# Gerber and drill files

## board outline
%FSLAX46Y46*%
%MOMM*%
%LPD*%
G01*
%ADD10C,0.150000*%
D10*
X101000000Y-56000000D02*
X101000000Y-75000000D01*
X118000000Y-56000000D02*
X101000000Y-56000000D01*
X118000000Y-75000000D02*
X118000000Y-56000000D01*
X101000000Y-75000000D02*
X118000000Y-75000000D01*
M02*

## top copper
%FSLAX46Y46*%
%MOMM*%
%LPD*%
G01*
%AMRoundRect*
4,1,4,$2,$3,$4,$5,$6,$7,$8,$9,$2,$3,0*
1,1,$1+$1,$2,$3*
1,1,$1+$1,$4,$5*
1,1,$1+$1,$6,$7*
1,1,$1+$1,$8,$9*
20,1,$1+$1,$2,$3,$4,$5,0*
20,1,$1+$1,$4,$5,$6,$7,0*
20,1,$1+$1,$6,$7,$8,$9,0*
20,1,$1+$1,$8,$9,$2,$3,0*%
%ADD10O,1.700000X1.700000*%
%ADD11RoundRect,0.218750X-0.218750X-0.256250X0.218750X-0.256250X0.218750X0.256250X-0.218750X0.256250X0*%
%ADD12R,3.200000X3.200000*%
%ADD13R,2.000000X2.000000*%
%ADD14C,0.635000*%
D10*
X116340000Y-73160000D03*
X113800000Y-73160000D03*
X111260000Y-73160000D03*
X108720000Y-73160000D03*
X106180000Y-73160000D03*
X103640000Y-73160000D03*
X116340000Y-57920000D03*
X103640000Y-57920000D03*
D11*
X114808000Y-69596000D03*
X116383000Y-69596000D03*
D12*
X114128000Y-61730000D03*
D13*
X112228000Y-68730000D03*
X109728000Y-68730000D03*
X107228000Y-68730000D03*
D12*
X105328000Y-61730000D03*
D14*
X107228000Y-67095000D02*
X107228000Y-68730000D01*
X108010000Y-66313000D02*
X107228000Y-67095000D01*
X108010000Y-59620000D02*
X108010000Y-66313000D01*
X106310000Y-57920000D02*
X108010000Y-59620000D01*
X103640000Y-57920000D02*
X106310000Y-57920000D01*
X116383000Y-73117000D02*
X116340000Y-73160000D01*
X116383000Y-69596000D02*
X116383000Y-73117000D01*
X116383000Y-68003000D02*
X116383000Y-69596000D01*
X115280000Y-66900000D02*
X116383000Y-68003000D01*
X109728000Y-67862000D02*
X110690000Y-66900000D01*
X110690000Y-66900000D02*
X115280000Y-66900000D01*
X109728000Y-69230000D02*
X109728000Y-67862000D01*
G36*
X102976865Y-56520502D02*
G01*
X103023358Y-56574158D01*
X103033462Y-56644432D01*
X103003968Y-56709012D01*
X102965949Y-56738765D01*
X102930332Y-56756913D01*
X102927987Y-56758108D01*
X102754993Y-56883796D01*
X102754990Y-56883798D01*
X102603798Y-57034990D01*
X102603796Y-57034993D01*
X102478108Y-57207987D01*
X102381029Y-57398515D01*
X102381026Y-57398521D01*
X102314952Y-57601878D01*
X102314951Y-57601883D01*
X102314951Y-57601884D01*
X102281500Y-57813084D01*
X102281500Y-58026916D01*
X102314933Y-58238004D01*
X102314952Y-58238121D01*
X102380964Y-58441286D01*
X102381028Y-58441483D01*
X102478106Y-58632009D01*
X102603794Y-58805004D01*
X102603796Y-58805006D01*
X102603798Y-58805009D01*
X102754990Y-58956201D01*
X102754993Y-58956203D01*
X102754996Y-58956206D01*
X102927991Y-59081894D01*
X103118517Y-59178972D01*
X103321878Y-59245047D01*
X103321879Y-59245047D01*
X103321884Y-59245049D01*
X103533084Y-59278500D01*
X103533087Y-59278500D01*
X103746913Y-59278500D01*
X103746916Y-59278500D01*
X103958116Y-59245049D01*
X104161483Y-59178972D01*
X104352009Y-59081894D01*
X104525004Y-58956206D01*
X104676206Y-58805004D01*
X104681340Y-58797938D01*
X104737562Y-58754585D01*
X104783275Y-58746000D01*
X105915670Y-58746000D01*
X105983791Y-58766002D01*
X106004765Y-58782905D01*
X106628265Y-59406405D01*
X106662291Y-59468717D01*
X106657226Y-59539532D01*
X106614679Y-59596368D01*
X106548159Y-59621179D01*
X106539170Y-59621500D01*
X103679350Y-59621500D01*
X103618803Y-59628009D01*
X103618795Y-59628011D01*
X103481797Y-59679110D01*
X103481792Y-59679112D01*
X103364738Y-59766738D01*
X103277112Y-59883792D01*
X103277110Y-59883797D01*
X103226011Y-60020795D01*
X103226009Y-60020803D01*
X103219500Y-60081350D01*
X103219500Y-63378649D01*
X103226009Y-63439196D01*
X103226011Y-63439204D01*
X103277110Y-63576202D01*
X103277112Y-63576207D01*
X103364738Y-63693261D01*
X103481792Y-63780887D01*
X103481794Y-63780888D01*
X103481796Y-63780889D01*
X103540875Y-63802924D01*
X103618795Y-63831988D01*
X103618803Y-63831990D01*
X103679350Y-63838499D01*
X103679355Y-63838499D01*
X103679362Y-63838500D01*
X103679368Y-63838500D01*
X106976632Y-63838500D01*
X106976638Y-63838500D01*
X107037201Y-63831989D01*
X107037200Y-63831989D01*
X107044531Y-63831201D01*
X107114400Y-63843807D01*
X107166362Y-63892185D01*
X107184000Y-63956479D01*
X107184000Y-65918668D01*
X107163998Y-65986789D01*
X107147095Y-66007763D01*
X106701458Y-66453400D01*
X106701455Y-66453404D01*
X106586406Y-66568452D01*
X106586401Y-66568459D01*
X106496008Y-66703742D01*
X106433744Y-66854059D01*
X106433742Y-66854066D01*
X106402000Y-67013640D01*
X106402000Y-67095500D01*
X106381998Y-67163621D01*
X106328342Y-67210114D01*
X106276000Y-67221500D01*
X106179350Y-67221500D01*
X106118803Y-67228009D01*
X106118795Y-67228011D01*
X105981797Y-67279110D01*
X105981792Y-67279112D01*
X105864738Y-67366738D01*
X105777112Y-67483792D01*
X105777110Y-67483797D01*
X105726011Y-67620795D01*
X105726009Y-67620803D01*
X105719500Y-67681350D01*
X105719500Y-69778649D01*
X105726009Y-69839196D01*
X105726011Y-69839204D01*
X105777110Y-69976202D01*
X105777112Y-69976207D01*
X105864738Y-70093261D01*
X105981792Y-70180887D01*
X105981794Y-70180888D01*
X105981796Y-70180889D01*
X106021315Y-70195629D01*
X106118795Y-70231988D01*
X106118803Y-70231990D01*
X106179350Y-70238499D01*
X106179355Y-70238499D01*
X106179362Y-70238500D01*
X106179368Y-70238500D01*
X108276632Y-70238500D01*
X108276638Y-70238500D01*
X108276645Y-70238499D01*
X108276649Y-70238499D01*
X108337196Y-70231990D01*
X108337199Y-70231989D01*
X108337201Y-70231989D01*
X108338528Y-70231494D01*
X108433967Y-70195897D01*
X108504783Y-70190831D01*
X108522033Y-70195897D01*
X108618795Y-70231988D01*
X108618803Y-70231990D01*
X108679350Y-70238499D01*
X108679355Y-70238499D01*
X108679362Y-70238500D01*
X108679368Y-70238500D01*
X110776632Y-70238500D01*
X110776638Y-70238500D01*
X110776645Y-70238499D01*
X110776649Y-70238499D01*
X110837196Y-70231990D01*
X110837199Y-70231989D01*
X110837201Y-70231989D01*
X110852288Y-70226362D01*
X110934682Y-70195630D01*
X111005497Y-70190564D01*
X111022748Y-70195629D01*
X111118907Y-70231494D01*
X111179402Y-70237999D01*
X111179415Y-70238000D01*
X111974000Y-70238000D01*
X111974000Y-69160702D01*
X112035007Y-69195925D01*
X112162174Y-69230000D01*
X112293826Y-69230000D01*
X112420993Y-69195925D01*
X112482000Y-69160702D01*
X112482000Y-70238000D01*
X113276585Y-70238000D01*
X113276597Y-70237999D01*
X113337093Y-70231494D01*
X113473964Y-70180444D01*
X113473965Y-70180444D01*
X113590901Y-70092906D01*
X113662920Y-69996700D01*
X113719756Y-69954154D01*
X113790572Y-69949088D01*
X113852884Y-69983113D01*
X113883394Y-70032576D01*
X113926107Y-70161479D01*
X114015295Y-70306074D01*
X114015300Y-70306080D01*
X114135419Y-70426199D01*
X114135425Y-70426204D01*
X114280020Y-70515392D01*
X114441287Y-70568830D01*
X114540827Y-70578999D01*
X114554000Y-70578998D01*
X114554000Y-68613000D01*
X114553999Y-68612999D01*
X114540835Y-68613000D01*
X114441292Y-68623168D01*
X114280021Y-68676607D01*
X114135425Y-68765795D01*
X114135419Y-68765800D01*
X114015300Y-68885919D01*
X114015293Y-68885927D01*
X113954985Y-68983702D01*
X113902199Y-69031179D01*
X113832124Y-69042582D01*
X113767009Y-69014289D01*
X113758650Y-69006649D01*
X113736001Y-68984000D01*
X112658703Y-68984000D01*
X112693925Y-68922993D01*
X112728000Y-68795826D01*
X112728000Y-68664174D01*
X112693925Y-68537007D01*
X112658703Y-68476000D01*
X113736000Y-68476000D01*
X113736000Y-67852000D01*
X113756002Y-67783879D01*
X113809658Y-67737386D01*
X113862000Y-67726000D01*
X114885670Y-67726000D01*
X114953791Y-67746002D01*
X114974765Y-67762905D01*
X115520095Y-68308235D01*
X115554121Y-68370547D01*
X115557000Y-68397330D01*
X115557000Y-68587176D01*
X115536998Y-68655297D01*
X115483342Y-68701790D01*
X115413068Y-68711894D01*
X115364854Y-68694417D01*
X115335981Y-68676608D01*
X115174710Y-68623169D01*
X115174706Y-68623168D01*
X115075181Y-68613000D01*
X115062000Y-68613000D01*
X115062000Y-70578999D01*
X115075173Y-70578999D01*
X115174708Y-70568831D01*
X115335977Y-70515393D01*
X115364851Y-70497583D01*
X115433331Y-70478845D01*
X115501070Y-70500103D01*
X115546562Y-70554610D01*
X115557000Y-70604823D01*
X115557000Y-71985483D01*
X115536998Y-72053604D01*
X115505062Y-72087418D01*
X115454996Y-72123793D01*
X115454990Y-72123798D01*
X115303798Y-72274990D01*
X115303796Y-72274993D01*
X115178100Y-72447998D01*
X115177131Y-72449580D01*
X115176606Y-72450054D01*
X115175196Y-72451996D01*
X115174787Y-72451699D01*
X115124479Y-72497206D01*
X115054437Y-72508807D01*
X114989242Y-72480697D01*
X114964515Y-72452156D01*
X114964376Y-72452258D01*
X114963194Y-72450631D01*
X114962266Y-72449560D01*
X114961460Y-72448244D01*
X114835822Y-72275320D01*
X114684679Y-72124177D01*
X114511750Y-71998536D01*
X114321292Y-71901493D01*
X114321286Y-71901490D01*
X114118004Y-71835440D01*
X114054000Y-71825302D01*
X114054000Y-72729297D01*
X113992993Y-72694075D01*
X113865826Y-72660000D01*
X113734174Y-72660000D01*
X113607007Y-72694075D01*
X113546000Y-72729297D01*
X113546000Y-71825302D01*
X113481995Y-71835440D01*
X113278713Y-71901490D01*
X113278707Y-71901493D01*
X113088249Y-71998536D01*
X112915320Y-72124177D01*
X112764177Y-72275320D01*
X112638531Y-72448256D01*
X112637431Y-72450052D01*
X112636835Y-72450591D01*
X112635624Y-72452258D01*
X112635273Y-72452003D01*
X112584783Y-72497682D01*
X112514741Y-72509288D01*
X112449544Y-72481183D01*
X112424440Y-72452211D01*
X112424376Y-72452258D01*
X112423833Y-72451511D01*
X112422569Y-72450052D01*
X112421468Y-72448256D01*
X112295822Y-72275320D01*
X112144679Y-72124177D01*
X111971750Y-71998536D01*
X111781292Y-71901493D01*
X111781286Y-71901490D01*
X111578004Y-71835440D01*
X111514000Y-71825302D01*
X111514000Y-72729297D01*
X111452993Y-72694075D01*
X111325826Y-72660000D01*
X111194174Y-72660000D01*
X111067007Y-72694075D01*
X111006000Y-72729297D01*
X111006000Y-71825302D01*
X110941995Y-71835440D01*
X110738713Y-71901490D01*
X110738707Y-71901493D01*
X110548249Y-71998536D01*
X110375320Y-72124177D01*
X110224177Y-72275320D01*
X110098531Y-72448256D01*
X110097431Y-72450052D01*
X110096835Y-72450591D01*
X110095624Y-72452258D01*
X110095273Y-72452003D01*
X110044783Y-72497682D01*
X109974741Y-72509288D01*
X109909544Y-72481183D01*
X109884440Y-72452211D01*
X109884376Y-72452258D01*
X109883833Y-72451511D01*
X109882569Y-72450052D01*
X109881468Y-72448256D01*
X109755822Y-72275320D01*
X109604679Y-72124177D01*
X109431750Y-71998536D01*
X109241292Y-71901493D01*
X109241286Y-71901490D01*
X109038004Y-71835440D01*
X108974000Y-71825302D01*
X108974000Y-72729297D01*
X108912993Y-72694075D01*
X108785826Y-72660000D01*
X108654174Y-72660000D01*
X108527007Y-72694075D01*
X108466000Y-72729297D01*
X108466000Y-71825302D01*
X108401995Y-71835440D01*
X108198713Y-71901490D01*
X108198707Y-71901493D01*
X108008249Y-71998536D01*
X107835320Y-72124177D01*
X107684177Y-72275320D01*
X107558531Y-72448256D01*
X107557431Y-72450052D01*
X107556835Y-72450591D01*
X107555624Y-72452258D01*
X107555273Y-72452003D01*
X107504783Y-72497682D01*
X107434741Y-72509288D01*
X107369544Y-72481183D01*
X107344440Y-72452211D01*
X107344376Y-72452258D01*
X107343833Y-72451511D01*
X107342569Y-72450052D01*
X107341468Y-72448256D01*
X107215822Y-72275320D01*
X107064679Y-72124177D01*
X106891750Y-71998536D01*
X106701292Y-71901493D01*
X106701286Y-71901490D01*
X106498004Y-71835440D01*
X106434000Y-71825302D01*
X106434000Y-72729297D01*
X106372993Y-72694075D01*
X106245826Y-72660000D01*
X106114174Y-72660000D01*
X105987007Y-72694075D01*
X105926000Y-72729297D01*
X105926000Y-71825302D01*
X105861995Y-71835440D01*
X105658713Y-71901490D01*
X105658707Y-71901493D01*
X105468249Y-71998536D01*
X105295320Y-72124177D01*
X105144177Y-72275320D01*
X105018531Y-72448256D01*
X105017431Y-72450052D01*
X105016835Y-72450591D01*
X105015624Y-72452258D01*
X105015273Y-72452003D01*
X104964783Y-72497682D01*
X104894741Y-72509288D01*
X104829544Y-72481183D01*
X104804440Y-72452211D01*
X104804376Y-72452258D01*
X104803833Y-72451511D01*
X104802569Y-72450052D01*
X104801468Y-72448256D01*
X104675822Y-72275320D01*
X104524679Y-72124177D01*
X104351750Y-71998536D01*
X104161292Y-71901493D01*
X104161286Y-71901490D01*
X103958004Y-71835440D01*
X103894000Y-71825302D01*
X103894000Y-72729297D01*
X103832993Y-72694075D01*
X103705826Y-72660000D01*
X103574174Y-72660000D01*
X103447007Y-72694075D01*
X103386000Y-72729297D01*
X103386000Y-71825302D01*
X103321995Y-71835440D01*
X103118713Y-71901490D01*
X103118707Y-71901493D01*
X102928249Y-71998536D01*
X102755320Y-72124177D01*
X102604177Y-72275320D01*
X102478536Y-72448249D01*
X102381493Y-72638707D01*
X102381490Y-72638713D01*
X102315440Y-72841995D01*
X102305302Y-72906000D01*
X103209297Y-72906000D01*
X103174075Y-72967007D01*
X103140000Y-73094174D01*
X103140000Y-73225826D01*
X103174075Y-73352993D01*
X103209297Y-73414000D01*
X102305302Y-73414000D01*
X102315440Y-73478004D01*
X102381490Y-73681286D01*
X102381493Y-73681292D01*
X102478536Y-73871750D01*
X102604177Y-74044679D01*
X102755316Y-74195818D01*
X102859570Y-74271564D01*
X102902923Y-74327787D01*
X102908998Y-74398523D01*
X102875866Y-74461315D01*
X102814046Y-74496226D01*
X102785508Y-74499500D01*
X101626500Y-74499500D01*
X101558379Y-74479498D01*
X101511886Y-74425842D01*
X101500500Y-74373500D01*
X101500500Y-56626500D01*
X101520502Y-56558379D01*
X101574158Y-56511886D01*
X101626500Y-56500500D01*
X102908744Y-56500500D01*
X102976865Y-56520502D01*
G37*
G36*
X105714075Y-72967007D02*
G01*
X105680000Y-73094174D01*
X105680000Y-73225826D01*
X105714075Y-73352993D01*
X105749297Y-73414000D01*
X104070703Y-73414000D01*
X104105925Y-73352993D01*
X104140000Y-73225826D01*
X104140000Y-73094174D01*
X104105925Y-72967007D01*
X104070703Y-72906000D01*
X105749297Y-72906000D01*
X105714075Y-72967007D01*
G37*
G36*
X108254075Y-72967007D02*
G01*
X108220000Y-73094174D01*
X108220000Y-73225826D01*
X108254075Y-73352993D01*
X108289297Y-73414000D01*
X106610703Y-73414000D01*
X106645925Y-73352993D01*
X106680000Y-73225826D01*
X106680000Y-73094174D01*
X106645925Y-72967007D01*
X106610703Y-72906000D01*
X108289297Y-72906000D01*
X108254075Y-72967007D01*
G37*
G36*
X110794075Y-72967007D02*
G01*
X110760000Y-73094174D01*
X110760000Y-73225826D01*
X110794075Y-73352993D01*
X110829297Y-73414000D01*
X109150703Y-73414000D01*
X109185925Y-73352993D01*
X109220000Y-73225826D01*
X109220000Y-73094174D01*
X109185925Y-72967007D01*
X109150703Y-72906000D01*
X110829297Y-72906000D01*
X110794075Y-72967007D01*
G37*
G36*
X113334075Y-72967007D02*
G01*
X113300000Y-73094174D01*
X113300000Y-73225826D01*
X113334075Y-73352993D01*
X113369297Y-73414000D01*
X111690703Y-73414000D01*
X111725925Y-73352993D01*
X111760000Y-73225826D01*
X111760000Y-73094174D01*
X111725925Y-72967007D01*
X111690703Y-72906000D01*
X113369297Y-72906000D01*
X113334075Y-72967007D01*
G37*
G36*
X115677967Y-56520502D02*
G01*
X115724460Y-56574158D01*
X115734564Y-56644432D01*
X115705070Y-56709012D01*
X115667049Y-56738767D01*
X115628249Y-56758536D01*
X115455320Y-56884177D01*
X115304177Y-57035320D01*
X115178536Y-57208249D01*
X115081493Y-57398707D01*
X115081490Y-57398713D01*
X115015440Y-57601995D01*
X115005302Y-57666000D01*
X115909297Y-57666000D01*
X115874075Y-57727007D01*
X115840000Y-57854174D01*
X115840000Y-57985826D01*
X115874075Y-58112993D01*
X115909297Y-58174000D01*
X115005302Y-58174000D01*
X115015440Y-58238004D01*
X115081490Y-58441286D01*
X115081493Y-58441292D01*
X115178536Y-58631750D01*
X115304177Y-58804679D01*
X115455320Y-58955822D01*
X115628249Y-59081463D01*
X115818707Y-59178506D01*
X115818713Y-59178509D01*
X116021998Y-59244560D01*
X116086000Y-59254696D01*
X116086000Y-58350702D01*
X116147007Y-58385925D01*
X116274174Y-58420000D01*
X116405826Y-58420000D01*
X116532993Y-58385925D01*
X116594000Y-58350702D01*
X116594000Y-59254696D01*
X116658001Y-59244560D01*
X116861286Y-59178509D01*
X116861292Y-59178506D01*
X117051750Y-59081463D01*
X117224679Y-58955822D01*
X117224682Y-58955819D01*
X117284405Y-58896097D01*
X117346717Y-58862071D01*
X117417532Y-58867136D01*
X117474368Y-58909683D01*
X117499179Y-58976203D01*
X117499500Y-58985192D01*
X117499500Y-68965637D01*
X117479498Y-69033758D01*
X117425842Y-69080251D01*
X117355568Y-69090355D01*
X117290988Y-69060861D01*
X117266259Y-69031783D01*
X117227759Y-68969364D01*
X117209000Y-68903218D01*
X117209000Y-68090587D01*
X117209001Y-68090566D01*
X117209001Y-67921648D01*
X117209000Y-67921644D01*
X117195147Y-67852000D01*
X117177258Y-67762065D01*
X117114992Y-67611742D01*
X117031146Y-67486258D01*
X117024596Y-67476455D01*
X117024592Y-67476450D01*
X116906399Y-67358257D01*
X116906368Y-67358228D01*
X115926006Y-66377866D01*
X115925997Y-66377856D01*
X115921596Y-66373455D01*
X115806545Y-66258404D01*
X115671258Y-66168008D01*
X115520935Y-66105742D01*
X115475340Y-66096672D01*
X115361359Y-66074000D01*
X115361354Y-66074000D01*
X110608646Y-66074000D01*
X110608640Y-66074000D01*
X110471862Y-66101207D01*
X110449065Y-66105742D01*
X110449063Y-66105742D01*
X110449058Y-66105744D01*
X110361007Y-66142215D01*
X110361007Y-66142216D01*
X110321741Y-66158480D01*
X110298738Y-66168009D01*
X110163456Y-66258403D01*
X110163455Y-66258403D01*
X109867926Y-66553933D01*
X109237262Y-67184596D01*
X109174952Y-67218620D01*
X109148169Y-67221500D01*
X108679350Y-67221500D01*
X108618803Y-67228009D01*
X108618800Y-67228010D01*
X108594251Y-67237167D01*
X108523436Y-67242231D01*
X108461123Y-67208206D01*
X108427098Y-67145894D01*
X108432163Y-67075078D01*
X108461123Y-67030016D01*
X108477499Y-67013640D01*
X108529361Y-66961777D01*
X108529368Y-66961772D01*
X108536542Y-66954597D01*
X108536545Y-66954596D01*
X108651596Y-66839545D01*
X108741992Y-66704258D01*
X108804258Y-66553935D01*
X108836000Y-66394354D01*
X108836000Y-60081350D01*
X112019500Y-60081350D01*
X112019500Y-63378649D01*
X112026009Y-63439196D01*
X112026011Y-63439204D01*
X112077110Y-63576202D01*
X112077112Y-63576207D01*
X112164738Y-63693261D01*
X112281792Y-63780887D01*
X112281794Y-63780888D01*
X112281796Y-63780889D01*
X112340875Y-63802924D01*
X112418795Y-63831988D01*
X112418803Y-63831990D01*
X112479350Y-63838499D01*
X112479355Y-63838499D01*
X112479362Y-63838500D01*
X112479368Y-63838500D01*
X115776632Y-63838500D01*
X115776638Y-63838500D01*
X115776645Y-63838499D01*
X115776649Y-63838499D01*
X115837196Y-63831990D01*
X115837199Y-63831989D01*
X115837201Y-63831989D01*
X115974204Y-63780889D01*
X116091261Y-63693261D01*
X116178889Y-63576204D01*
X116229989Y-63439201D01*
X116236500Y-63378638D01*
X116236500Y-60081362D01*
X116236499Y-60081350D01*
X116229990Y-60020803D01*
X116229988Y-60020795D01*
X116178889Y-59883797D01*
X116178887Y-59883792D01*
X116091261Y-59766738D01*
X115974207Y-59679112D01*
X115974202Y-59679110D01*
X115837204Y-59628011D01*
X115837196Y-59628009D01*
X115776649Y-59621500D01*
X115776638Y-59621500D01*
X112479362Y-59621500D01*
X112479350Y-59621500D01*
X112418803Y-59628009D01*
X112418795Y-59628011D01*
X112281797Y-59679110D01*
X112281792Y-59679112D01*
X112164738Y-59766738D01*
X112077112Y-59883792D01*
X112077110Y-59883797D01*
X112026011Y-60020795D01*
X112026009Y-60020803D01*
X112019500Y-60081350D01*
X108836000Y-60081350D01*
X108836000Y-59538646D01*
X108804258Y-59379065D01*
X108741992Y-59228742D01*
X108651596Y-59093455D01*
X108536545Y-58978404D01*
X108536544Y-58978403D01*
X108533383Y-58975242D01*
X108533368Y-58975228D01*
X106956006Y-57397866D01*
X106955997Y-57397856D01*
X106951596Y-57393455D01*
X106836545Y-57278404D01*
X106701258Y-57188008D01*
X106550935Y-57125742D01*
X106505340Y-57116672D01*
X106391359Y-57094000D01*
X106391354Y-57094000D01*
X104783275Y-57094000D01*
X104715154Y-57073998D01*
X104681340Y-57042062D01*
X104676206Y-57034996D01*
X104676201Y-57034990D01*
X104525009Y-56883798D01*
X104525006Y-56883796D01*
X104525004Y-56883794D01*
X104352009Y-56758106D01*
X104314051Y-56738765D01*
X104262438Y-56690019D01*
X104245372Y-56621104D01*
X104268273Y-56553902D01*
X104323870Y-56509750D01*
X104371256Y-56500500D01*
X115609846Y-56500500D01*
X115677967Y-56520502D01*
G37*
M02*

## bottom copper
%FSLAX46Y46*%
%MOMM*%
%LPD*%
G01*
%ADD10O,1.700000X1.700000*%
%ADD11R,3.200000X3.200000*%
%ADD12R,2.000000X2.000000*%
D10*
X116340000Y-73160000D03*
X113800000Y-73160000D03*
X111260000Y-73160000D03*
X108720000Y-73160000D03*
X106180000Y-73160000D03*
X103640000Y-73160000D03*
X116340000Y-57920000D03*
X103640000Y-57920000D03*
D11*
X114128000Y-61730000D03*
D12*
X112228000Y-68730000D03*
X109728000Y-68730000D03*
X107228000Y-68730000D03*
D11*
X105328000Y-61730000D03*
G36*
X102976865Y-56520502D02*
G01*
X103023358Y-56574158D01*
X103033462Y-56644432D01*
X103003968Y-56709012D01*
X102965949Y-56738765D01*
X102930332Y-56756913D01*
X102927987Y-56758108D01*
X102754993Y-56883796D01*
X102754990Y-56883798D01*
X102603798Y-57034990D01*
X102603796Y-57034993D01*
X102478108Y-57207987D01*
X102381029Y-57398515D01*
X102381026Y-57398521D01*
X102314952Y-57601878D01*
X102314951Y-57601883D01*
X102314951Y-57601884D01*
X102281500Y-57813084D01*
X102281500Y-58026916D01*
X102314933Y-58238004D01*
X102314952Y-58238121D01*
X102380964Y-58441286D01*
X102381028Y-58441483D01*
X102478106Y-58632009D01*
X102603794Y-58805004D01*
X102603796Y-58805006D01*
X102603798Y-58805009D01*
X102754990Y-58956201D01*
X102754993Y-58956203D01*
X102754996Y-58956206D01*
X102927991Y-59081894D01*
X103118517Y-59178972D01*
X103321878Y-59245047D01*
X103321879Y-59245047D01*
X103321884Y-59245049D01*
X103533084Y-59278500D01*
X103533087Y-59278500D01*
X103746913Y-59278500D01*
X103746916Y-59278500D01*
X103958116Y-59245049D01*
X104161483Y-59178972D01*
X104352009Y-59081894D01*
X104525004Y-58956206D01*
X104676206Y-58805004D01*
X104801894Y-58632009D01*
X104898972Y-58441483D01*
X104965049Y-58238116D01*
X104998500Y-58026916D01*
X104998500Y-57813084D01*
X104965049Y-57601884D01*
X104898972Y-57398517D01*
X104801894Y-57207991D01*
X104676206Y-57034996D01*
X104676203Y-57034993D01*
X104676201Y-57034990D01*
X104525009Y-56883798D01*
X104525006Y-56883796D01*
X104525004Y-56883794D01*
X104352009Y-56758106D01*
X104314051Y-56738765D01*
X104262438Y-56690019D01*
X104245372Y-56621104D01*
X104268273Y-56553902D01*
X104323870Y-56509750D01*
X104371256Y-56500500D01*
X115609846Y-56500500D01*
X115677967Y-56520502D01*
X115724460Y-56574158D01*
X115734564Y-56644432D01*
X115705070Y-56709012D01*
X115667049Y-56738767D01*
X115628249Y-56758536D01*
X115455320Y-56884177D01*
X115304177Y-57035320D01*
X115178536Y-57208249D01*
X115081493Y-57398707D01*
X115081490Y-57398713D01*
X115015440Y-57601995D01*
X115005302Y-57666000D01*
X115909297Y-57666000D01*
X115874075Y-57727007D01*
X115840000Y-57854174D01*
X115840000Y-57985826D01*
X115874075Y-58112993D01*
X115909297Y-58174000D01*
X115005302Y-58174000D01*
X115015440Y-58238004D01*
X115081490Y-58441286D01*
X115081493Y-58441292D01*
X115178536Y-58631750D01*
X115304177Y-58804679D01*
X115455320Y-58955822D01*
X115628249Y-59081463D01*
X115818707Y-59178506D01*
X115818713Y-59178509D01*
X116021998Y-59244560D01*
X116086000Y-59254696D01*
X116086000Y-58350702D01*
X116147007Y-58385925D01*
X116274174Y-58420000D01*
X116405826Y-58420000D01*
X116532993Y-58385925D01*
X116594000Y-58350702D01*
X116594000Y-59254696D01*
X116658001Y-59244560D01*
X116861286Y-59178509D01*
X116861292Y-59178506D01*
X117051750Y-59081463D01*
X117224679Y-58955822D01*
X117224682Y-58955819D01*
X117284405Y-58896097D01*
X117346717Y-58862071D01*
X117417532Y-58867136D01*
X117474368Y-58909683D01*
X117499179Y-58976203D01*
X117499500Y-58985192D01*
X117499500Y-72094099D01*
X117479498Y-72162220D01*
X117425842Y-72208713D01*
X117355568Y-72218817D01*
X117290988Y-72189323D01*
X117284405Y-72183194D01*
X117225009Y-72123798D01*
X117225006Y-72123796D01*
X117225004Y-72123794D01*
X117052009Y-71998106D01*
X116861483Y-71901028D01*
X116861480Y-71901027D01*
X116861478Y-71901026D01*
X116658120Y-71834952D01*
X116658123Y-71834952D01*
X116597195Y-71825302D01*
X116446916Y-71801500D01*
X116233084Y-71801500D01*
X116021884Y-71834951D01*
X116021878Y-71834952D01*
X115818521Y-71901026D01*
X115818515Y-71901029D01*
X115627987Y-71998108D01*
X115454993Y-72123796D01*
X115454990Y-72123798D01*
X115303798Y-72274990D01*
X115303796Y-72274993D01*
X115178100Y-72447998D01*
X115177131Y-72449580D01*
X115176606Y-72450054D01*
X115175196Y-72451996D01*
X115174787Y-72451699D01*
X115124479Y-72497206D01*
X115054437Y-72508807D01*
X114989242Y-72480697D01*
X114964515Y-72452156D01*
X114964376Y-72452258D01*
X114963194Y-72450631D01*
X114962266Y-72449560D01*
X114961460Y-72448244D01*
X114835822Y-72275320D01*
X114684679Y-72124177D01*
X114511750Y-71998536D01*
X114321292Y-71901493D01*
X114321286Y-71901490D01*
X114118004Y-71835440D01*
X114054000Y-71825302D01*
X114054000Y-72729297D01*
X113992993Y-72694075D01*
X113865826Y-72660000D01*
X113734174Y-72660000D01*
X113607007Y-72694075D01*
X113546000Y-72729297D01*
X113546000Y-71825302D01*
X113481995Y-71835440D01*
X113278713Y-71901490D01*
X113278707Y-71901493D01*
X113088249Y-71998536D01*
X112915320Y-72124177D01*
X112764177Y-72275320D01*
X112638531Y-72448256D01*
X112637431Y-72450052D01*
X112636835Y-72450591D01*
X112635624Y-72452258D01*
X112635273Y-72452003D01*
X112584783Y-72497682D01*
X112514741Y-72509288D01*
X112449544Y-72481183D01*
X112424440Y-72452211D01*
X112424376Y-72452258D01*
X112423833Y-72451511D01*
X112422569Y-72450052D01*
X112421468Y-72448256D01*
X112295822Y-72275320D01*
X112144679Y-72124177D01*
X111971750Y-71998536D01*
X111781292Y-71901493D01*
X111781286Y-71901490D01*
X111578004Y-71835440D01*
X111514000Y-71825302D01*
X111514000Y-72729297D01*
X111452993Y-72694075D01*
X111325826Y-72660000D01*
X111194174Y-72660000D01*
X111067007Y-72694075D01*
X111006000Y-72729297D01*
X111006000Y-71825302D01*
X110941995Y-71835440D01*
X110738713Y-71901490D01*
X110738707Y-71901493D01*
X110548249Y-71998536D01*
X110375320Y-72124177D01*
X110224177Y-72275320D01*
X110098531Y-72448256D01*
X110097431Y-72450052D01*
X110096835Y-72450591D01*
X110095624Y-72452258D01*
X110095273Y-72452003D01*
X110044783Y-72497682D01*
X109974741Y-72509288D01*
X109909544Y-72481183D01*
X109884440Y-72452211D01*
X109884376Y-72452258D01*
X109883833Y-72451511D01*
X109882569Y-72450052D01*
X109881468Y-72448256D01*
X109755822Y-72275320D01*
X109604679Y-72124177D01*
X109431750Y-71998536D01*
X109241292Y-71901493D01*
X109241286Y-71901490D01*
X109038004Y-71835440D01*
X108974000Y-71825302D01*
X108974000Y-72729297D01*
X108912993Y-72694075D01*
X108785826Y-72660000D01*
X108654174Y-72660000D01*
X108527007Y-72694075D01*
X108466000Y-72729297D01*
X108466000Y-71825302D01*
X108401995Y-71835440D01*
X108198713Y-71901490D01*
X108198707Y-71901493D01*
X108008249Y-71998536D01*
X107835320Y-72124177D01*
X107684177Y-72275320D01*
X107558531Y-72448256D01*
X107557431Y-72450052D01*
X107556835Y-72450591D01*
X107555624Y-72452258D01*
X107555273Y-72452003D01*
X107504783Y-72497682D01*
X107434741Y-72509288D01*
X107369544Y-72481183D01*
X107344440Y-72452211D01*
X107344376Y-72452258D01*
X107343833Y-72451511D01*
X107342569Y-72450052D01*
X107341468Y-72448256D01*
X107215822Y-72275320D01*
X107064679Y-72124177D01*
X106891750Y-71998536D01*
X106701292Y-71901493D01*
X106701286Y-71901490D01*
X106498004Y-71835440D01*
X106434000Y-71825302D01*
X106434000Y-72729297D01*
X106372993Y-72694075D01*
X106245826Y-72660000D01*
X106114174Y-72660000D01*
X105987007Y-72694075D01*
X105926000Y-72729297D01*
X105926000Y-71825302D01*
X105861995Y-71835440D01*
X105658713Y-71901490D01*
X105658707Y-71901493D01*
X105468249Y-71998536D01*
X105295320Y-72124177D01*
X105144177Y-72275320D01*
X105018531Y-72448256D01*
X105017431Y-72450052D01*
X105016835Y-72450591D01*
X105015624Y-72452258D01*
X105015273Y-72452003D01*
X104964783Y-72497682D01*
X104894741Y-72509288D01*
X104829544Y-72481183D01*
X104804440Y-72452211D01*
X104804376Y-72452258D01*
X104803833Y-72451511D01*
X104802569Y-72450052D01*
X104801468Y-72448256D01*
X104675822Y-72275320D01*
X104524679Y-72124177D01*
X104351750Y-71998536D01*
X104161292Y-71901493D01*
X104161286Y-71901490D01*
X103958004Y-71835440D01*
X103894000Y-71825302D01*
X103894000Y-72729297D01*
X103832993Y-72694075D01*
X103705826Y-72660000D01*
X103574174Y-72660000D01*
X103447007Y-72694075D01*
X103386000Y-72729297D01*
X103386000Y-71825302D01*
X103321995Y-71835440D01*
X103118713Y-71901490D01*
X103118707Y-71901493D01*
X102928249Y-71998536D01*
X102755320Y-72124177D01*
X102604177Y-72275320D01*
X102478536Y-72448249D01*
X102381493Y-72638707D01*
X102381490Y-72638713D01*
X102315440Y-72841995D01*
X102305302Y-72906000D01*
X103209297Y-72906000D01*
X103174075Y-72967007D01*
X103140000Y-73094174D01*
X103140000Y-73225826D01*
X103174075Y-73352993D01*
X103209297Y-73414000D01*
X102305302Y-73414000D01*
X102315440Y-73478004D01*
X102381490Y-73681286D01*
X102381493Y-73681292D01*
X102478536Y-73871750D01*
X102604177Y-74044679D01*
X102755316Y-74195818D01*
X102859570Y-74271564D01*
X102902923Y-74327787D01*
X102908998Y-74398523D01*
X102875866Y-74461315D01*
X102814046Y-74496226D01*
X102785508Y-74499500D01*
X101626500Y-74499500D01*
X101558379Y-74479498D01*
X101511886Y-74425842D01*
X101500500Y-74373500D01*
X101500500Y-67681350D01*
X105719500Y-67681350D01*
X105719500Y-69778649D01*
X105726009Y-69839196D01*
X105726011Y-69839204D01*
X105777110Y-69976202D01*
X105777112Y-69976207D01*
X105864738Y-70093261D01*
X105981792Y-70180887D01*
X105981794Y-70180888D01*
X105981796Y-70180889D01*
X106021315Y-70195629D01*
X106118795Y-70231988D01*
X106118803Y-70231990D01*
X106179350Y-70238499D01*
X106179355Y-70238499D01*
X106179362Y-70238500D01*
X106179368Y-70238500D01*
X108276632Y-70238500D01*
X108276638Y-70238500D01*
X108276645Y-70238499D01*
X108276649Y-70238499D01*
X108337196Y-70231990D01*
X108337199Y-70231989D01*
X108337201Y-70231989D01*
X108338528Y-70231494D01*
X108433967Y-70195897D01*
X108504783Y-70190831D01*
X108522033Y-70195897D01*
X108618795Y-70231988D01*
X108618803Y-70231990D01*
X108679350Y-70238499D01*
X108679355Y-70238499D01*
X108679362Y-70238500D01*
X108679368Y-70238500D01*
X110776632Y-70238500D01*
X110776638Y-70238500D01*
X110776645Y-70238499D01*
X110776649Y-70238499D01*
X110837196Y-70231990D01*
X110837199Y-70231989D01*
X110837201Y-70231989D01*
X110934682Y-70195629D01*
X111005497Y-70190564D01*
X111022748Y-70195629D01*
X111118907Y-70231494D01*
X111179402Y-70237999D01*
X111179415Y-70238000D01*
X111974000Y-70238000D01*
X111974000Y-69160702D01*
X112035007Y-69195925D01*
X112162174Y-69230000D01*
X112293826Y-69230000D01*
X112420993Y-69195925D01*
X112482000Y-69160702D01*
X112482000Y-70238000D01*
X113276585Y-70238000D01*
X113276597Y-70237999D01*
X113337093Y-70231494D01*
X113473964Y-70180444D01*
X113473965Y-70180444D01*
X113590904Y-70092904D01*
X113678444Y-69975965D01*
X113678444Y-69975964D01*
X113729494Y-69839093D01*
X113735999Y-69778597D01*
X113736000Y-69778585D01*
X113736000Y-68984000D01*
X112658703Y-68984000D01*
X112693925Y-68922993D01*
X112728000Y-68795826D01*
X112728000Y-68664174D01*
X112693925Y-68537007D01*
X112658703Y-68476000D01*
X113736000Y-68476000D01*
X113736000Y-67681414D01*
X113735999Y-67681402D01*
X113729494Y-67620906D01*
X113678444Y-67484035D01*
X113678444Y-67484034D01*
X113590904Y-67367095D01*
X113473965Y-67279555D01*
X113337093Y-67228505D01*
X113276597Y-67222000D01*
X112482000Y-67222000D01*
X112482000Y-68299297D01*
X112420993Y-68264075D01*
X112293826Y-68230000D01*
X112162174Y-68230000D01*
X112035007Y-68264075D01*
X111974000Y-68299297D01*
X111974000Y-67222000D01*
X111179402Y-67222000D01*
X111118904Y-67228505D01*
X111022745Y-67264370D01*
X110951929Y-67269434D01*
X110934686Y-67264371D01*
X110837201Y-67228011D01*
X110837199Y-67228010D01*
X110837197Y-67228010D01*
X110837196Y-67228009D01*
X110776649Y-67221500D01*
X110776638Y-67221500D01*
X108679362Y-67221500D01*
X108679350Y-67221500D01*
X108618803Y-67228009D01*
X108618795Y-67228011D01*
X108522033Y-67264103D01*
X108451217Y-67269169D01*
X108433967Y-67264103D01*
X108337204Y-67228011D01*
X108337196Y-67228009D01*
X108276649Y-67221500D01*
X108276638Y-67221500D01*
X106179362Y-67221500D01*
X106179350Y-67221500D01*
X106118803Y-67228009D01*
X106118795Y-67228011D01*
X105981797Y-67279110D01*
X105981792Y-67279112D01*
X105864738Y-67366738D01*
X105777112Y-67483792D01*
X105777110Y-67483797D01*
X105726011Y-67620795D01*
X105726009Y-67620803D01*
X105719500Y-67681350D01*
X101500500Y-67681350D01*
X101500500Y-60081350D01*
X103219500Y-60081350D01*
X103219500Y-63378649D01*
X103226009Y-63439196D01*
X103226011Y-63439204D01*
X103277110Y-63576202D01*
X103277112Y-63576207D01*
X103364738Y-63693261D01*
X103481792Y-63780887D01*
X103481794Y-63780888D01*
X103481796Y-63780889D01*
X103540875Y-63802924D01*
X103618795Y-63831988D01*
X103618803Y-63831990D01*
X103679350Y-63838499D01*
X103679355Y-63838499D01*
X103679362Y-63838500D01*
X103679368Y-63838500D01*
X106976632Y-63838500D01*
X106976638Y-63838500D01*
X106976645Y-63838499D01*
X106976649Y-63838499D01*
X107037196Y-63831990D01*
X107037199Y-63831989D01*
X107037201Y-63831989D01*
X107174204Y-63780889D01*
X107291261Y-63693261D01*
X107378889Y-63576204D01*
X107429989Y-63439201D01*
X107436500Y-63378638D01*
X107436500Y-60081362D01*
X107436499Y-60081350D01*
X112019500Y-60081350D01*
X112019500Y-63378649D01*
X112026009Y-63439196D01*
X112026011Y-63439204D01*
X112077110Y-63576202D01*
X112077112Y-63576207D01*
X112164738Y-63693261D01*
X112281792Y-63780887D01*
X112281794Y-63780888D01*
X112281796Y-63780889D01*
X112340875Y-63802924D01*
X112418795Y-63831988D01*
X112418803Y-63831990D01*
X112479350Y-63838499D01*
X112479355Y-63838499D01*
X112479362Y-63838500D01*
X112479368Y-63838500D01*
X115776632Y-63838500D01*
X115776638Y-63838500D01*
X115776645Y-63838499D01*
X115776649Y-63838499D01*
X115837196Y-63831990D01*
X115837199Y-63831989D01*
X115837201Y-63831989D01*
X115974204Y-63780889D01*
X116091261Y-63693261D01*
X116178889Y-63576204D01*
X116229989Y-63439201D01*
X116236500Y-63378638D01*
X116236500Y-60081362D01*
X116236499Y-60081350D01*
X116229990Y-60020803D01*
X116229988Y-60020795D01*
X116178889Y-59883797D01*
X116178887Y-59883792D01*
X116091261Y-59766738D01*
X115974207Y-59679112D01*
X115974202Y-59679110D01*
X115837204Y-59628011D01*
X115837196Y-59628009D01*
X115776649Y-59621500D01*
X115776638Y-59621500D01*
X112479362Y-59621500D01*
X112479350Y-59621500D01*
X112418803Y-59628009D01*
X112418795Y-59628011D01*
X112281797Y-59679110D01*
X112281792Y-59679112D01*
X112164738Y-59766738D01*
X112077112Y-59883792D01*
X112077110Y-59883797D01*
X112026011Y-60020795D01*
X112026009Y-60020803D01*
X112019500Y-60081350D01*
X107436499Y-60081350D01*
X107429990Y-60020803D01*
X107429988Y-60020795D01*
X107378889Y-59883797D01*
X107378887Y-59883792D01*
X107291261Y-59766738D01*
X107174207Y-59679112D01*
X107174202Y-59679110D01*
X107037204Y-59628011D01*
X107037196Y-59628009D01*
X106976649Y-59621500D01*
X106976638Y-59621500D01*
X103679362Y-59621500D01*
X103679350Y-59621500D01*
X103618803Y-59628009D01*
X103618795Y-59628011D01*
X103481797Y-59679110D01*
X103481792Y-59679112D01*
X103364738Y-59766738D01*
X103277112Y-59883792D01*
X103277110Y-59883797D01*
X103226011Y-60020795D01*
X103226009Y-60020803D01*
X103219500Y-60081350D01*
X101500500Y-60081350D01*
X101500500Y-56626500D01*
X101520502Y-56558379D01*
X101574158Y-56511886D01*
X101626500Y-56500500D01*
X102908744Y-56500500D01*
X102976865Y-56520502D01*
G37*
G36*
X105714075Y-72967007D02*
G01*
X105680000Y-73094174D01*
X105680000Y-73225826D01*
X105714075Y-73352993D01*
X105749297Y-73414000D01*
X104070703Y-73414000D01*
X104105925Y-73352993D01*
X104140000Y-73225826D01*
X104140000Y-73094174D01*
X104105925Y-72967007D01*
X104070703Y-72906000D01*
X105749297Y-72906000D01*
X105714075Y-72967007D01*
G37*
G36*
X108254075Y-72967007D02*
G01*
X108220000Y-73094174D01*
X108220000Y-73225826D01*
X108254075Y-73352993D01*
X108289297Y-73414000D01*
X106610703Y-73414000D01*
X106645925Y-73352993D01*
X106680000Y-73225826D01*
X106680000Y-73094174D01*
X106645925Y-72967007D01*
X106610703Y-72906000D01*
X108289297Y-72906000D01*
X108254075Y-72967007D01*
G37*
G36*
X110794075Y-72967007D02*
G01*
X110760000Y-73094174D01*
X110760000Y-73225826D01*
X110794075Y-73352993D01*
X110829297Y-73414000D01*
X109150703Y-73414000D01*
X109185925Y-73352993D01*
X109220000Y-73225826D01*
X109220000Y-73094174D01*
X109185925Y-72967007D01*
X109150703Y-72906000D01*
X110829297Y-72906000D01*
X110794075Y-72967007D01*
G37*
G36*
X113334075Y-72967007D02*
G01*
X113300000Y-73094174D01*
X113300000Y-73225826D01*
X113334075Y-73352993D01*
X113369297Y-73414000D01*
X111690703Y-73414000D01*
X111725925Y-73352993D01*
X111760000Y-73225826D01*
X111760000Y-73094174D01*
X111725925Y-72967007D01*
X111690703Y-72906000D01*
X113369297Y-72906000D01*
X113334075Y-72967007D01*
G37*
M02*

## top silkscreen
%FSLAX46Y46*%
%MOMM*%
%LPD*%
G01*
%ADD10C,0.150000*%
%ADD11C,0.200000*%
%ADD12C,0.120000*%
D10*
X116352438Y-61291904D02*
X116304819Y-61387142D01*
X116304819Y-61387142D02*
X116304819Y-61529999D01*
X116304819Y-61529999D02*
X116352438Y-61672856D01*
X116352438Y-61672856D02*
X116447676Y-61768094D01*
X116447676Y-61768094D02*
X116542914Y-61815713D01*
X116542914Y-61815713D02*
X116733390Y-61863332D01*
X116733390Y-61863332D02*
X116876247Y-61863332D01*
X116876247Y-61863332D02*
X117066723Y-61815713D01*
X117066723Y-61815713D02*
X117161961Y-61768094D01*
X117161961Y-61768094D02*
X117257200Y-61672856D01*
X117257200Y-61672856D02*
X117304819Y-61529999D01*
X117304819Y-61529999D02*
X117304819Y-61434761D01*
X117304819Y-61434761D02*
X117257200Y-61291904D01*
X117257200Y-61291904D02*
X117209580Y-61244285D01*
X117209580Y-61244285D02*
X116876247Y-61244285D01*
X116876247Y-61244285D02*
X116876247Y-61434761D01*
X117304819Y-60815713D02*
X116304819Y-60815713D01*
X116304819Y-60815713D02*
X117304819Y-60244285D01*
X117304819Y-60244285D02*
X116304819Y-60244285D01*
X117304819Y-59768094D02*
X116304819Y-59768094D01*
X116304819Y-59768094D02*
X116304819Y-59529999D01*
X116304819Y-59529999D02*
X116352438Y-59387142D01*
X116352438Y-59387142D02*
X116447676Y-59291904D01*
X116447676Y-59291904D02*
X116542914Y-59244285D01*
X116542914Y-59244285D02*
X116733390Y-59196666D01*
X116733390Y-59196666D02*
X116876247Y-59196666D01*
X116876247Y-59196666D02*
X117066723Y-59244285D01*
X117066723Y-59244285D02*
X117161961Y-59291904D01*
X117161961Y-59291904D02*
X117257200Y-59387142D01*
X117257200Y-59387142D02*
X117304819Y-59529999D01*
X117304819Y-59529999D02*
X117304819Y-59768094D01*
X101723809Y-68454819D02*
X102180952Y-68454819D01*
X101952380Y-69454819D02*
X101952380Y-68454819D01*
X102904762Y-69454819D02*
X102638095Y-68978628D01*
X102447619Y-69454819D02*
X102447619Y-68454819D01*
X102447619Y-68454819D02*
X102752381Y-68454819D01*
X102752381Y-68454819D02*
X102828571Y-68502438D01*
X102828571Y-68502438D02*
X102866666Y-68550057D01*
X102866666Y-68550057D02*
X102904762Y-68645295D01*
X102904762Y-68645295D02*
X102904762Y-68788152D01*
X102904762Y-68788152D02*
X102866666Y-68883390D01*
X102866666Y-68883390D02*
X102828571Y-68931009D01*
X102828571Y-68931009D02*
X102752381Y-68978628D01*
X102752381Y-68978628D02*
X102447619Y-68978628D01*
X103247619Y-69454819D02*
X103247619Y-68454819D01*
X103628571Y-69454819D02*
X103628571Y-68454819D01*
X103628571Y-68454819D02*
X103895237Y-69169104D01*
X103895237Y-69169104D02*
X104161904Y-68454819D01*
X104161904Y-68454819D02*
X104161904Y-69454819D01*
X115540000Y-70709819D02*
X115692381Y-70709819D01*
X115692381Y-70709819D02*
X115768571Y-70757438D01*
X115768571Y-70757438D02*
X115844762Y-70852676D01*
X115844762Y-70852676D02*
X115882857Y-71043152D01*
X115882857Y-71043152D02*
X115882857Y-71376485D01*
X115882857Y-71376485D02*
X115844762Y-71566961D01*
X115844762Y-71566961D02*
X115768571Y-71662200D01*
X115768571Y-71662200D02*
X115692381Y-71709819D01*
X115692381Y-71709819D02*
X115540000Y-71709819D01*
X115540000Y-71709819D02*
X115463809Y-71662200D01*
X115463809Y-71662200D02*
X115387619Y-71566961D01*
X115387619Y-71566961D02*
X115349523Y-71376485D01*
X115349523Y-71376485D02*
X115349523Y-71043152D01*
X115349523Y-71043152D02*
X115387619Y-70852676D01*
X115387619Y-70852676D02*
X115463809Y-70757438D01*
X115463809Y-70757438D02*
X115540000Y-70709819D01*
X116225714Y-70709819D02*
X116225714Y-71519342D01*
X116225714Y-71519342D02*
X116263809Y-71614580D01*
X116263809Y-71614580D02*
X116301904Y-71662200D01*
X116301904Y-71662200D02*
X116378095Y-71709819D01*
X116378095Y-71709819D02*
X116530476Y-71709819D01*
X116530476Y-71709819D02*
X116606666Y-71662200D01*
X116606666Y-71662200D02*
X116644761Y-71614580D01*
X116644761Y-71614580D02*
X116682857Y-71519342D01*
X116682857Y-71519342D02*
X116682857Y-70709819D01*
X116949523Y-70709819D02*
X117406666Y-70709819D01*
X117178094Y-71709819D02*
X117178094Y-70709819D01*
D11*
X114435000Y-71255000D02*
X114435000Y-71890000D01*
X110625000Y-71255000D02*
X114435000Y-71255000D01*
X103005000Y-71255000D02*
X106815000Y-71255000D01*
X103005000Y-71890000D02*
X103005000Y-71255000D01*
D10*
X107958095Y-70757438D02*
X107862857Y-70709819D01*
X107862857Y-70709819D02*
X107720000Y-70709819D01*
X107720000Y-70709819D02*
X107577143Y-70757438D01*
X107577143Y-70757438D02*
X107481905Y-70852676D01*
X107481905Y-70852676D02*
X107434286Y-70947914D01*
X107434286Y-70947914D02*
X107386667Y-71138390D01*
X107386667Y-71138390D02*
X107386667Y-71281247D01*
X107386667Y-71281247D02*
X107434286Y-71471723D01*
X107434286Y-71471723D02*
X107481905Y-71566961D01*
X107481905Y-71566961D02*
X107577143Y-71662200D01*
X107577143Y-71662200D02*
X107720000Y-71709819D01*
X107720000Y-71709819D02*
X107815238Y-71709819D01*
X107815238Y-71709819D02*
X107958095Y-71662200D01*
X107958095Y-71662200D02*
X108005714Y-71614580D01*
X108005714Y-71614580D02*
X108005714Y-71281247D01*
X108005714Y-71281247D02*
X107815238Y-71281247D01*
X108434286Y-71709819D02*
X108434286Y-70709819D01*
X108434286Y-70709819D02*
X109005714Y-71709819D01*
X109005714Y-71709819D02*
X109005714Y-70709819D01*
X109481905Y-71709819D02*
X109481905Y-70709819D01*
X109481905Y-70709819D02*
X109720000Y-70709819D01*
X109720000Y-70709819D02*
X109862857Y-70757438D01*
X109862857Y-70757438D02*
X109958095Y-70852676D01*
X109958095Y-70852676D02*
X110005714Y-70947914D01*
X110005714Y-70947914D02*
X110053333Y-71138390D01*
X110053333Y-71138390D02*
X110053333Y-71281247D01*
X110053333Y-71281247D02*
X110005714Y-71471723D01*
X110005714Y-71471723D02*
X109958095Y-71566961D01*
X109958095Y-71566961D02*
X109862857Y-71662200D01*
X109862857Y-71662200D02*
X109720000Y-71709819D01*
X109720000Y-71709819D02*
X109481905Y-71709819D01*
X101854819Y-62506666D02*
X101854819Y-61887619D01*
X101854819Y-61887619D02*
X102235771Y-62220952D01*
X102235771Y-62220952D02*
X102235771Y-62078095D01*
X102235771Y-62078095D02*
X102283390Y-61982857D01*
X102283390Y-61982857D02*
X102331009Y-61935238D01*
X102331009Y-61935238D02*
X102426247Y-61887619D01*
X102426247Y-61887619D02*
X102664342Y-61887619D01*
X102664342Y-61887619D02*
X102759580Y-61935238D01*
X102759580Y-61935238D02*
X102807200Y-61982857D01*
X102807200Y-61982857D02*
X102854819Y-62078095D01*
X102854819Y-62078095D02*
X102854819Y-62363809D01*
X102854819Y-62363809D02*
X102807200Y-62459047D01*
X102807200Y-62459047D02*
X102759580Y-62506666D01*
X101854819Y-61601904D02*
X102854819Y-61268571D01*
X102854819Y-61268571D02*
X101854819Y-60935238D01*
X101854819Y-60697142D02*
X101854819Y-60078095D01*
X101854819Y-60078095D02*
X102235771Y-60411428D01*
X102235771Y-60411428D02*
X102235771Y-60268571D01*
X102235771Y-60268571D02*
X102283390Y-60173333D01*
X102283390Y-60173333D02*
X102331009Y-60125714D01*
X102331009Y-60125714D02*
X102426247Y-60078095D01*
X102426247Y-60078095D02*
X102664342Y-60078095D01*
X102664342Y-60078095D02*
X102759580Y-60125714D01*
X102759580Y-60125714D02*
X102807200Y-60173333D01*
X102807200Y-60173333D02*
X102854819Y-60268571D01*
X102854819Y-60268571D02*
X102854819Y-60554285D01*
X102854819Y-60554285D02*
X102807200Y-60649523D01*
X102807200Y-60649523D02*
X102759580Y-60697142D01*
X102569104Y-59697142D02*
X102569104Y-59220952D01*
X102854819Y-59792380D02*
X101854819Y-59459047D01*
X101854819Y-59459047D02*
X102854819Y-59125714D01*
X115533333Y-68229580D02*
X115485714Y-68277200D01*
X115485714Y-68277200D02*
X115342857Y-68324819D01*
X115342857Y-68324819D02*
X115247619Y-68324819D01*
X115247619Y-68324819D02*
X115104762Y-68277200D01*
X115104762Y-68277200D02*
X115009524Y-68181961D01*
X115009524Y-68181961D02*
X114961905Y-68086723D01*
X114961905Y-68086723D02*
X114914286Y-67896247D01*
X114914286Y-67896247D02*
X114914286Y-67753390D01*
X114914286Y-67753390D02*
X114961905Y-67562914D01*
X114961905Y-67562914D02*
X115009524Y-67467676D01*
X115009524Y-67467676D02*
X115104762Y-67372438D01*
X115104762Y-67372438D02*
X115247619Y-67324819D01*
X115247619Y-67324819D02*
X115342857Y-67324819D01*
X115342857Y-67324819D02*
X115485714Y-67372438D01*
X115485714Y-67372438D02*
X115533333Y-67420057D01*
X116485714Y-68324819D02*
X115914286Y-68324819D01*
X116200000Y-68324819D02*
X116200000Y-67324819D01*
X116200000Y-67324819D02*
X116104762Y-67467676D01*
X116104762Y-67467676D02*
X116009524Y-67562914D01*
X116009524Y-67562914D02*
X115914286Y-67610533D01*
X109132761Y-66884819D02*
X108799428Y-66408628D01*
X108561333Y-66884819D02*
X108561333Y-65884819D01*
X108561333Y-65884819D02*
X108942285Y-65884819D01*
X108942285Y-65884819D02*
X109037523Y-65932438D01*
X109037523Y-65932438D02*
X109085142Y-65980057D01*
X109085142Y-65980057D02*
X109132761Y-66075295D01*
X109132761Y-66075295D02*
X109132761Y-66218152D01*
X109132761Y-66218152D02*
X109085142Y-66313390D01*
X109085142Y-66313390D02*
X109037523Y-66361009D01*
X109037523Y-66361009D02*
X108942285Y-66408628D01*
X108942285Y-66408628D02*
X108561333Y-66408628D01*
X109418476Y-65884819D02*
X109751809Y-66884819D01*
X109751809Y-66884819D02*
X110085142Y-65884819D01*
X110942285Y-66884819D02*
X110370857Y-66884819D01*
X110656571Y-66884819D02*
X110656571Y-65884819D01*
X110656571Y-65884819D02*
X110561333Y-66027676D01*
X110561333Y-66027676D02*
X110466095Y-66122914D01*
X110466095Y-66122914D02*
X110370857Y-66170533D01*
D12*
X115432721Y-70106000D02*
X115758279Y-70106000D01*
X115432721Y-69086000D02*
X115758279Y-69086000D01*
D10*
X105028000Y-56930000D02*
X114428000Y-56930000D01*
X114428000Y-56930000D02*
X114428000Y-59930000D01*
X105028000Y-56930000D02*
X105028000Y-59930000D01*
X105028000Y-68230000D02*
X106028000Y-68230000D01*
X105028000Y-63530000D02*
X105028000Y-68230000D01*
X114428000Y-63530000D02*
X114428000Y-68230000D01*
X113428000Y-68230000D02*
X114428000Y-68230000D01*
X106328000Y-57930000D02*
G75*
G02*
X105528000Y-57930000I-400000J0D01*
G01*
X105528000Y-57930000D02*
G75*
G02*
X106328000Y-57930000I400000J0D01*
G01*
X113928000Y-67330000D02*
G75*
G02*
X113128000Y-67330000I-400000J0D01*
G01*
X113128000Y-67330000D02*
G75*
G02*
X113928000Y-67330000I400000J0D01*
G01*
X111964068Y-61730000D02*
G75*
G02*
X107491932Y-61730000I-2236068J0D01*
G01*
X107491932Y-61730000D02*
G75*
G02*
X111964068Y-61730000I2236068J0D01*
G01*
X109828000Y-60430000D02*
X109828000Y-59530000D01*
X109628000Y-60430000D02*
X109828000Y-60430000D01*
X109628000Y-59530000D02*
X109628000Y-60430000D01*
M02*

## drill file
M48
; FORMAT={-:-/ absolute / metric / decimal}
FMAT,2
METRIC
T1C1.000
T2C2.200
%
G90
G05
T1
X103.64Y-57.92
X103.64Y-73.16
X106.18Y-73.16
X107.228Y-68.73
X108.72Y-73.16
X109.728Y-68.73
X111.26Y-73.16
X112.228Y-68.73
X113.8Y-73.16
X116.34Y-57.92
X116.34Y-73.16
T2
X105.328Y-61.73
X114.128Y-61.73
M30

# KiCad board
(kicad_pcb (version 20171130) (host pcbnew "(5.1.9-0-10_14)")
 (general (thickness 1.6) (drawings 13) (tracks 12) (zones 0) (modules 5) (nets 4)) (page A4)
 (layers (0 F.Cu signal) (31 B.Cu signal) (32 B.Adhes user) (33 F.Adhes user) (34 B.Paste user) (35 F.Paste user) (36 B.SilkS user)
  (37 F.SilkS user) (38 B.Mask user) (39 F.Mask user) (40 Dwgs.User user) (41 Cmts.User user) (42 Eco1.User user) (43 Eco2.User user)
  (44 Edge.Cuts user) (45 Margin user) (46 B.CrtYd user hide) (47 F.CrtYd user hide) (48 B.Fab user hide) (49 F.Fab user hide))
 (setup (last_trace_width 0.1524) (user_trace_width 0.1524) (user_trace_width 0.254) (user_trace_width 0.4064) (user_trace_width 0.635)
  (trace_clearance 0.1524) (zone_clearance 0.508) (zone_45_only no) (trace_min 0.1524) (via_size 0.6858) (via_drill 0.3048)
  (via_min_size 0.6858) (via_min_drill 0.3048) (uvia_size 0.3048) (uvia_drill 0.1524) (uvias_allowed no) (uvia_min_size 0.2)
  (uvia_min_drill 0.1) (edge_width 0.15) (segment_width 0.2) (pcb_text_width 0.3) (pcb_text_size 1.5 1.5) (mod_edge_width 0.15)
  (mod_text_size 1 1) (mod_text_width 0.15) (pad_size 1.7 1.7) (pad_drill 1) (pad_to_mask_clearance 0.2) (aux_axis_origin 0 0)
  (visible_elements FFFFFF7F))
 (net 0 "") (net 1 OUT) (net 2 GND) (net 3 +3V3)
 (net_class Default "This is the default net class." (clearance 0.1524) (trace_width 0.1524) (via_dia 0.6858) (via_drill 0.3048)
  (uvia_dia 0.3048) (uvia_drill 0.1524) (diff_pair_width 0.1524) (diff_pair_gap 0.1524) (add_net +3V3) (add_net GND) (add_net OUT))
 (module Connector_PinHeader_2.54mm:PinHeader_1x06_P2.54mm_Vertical (layer B.Cu) (at 116.34 73.16 90)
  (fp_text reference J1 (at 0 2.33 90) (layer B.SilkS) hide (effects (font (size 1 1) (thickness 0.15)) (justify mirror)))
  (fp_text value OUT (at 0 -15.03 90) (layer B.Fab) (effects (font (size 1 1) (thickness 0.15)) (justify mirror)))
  (pad 1 thru_hole oval (at 0 0 90) (size 1.7 1.7) (drill 1) (layers *.Cu *.Mask) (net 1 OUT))
  (pad 2 thru_hole oval (at 0 -2.54 90) (size 1.7 1.7) (drill 1) (layers *.Cu *.Mask) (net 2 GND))
  (pad 3 thru_hole oval (at 0 -5.08 90) (size 1.7 1.7) (drill 1) (layers *.Cu *.Mask) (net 2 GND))
  (pad 4 thru_hole oval (at 0 -7.62 90) (size 1.7 1.7) (drill 1) (layers *.Cu *.Mask) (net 2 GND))
  (pad 5 thru_hole oval (at 0 -10.16 90) (size 1.7 1.7) (drill 1) (layers *.Cu *.Mask) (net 2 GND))
  (pad 6 thru_hole oval (at 0 -12.7 90) (size 1.7 1.7) (drill 1) (layers *.Cu *.Mask) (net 2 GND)))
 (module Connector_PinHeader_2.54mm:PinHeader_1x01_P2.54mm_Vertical (layer B.Cu) (at 116.34 57.92 90)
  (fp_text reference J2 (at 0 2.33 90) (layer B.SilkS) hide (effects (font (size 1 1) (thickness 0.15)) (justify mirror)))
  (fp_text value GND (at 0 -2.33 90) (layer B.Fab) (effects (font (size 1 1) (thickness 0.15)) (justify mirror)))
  (pad 1 thru_hole oval (at 0 0 90) (size 1.7 1.7) (drill 1) (layers *.Cu *.Mask) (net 2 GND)))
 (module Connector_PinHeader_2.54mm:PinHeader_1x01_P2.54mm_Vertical (layer B.Cu) (at 103.64 57.92 270)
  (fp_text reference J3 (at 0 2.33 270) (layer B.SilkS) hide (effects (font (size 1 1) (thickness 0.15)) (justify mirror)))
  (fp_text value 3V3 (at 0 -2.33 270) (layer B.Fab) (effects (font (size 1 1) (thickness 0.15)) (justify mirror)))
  (pad 1 thru_hole oval (at 0 0 270) (size 1.7 1.7) (drill 1) (layers *.Cu *.Mask) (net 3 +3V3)))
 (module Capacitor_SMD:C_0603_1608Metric (layer F.Cu) (at 115.5955 69.596)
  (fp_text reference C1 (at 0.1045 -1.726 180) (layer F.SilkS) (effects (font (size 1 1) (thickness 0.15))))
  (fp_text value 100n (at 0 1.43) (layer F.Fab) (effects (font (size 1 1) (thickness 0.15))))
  (fp_line (start -0.162779 0.51) (end 0.162779 0.51) (layer F.SilkS) (width 0.12))
  (fp_line (start -0.162779 -0.51) (end 0.162779 -0.51) (layer F.SilkS) (width 0.12))
  (pad 1 smd roundrect (at -0.7875 0) (size 0.875 0.95) (layers F.Cu F.Paste F.Mask) (roundrect_rratio 0.25) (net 2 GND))
  (pad 2 smd roundrect (at 0.7875 0) (size 0.875 0.95) (layers F.Cu F.Paste F.Mask) (roundrect_rratio 0.25) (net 1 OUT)))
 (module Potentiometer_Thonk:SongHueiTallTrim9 (layer F.Cu) (at 109.728 61.73)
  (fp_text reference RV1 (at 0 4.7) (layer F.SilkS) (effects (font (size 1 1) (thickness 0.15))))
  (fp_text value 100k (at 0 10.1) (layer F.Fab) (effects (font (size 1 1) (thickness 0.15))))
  (fp_line (start -4.7 -4.8) (end 4.7 -4.8) (layer F.SilkS) (width 0.15))
  (fp_line (start 4.7 -4.8) (end 4.7 -1.8) (layer F.SilkS) (width 0.15))
  (fp_line (start -4.7 -4.8) (end -4.7 -1.8) (layer F.SilkS) (width 0.15))
  (fp_line (start -4.7 6.5) (end -3.7 6.5) (layer F.SilkS) (width 0.15))
  (fp_line (start -4.7 1.8) (end -4.7 6.5) (layer F.SilkS) (width 0.15))
  (fp_line (start 4.7 1.8) (end 4.7 6.5) (layer F.SilkS) (width 0.15))
  (fp_line (start 3.7 6.5) (end 4.7 6.5) (layer F.SilkS) (width 0.15))
  (fp_circle (center -3.8 -3.8) (end -4.2 -3.8) (layer F.SilkS) (width 0.15))
  (fp_circle (center 3.8 5.6) (end 4.2 5.6) (layer F.SilkS) (width 0.15))
  (fp_circle (center 0 0) (end 2.2 0.4) (layer F.SilkS) (width 0.15))
  (fp_line (start 0.1 -1.3) (end 0.1 -2.2) (layer F.SilkS) (width 0.15))
  (fp_line (start -0.1 -1.3) (end 0.1 -1.3) (layer F.SilkS) (width 0.15))
  (fp_line (start -0.1 -2.2) (end -0.1 -1.3) (layer F.SilkS) (width 0.15))
  (pad "" thru_hole rect (at 4.4 0) (size 3.2 3.2) (drill 2.2) (layers *.Cu *.Mask))
  (pad 3 thru_hole rect (at 2.5 7) (size 2 2) (drill 1) (layers *.Cu *.Mask) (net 2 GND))
  (pad 2 thru_hole rect (at 0 7) (size 2 2) (drill 1) (layers *.Cu *.Mask) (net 1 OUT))
  (pad 1 thru_hole rect (at -2.5 7) (size 2 2) (drill 1) (layers *.Cu *.Mask) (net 3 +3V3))
  (pad "" thru_hole rect (at -4.4 0) (size 3.2 3.2) (drill 2.2) (layers *.Cu *.Mask)))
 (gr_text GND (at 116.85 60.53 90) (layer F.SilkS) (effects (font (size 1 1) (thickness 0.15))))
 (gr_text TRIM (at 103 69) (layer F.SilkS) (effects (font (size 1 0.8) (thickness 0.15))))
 (gr_line (start 101 56) (end 101 75) (layer Edge.Cuts) (width 0.15))
 (gr_line (start 118 56) (end 101 56) (layer Edge.Cuts) (width 0.15))
 (gr_line (start 118 75) (end 118 56) (layer Edge.Cuts) (width 0.15))
 (gr_line (start 101 75) (end 118 75) (layer Edge.Cuts) (width 0.15))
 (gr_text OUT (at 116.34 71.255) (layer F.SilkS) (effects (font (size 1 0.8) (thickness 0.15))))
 (gr_line (start 114.435 71.255) (end 114.435 71.89) (layer F.SilkS) (width 0.2))
 (gr_line (start 110.625 71.255) (end 114.435 71.255) (layer F.SilkS) (width 0.2))
 (gr_line (start 103.005 71.255) (end 106.815 71.255) (layer F.SilkS) (width 0.2))
 (gr_line (start 103.005 71.89) (end 103.005 71.255) (layer F.SilkS) (width 0.2))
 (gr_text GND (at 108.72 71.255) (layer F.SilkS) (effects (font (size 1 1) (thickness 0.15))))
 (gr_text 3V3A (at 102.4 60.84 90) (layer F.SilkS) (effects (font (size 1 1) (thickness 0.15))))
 (segment (start 107.228 67.095) (end 107.228 68.73) (width 0.635) (layer F.Cu) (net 3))
 (segment (start 108.01 66.313) (end 107.228 67.095) (width 0.635) (layer F.Cu) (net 3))
 (segment (start 108.01 59.62) (end 108.01 66.313) (width 0.635) (layer F.Cu) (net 3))
 (segment (start 106.31 57.92) (end 108.01 59.62) (width 0.635) (layer F.Cu) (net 3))
 (segment (start 103.64 57.92) (end 106.31 57.92) (width 0.635) (layer F.Cu) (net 3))
 (segment (start 116.383 73.117) (end 116.34 73.16) (width 0.635) (layer F.Cu) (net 1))
 (segment (start 116.383 69.596) (end 116.383 73.117) (width 0.635) (layer F.Cu) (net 1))
 (segment (start 116.383 68.003) (end 116.383 69.596) (width 0.635) (layer F.Cu) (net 1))
 (segment (start 115.28 66.9) (end 116.383 68.003) (width 0.635) (layer F.Cu) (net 1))
 (segment (start 109.728 67.862) (end 110.69 66.9) (width 0.635) (layer F.Cu) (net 1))
 (segment (start 110.69 66.9) (end 115.28 66.9) (width 0.635) (layer F.Cu) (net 1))
 (segment (start 109.728 69.23) (end 109.728 67.862) (width 0.635) (layer F.Cu) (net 1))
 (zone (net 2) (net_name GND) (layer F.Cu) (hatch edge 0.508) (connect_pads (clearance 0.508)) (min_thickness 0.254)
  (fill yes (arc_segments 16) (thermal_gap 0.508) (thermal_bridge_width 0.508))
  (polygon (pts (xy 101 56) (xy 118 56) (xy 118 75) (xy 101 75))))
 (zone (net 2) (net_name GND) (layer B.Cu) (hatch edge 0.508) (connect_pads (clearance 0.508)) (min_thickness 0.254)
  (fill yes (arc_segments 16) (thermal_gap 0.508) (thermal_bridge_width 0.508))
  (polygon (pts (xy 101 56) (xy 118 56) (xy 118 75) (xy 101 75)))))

